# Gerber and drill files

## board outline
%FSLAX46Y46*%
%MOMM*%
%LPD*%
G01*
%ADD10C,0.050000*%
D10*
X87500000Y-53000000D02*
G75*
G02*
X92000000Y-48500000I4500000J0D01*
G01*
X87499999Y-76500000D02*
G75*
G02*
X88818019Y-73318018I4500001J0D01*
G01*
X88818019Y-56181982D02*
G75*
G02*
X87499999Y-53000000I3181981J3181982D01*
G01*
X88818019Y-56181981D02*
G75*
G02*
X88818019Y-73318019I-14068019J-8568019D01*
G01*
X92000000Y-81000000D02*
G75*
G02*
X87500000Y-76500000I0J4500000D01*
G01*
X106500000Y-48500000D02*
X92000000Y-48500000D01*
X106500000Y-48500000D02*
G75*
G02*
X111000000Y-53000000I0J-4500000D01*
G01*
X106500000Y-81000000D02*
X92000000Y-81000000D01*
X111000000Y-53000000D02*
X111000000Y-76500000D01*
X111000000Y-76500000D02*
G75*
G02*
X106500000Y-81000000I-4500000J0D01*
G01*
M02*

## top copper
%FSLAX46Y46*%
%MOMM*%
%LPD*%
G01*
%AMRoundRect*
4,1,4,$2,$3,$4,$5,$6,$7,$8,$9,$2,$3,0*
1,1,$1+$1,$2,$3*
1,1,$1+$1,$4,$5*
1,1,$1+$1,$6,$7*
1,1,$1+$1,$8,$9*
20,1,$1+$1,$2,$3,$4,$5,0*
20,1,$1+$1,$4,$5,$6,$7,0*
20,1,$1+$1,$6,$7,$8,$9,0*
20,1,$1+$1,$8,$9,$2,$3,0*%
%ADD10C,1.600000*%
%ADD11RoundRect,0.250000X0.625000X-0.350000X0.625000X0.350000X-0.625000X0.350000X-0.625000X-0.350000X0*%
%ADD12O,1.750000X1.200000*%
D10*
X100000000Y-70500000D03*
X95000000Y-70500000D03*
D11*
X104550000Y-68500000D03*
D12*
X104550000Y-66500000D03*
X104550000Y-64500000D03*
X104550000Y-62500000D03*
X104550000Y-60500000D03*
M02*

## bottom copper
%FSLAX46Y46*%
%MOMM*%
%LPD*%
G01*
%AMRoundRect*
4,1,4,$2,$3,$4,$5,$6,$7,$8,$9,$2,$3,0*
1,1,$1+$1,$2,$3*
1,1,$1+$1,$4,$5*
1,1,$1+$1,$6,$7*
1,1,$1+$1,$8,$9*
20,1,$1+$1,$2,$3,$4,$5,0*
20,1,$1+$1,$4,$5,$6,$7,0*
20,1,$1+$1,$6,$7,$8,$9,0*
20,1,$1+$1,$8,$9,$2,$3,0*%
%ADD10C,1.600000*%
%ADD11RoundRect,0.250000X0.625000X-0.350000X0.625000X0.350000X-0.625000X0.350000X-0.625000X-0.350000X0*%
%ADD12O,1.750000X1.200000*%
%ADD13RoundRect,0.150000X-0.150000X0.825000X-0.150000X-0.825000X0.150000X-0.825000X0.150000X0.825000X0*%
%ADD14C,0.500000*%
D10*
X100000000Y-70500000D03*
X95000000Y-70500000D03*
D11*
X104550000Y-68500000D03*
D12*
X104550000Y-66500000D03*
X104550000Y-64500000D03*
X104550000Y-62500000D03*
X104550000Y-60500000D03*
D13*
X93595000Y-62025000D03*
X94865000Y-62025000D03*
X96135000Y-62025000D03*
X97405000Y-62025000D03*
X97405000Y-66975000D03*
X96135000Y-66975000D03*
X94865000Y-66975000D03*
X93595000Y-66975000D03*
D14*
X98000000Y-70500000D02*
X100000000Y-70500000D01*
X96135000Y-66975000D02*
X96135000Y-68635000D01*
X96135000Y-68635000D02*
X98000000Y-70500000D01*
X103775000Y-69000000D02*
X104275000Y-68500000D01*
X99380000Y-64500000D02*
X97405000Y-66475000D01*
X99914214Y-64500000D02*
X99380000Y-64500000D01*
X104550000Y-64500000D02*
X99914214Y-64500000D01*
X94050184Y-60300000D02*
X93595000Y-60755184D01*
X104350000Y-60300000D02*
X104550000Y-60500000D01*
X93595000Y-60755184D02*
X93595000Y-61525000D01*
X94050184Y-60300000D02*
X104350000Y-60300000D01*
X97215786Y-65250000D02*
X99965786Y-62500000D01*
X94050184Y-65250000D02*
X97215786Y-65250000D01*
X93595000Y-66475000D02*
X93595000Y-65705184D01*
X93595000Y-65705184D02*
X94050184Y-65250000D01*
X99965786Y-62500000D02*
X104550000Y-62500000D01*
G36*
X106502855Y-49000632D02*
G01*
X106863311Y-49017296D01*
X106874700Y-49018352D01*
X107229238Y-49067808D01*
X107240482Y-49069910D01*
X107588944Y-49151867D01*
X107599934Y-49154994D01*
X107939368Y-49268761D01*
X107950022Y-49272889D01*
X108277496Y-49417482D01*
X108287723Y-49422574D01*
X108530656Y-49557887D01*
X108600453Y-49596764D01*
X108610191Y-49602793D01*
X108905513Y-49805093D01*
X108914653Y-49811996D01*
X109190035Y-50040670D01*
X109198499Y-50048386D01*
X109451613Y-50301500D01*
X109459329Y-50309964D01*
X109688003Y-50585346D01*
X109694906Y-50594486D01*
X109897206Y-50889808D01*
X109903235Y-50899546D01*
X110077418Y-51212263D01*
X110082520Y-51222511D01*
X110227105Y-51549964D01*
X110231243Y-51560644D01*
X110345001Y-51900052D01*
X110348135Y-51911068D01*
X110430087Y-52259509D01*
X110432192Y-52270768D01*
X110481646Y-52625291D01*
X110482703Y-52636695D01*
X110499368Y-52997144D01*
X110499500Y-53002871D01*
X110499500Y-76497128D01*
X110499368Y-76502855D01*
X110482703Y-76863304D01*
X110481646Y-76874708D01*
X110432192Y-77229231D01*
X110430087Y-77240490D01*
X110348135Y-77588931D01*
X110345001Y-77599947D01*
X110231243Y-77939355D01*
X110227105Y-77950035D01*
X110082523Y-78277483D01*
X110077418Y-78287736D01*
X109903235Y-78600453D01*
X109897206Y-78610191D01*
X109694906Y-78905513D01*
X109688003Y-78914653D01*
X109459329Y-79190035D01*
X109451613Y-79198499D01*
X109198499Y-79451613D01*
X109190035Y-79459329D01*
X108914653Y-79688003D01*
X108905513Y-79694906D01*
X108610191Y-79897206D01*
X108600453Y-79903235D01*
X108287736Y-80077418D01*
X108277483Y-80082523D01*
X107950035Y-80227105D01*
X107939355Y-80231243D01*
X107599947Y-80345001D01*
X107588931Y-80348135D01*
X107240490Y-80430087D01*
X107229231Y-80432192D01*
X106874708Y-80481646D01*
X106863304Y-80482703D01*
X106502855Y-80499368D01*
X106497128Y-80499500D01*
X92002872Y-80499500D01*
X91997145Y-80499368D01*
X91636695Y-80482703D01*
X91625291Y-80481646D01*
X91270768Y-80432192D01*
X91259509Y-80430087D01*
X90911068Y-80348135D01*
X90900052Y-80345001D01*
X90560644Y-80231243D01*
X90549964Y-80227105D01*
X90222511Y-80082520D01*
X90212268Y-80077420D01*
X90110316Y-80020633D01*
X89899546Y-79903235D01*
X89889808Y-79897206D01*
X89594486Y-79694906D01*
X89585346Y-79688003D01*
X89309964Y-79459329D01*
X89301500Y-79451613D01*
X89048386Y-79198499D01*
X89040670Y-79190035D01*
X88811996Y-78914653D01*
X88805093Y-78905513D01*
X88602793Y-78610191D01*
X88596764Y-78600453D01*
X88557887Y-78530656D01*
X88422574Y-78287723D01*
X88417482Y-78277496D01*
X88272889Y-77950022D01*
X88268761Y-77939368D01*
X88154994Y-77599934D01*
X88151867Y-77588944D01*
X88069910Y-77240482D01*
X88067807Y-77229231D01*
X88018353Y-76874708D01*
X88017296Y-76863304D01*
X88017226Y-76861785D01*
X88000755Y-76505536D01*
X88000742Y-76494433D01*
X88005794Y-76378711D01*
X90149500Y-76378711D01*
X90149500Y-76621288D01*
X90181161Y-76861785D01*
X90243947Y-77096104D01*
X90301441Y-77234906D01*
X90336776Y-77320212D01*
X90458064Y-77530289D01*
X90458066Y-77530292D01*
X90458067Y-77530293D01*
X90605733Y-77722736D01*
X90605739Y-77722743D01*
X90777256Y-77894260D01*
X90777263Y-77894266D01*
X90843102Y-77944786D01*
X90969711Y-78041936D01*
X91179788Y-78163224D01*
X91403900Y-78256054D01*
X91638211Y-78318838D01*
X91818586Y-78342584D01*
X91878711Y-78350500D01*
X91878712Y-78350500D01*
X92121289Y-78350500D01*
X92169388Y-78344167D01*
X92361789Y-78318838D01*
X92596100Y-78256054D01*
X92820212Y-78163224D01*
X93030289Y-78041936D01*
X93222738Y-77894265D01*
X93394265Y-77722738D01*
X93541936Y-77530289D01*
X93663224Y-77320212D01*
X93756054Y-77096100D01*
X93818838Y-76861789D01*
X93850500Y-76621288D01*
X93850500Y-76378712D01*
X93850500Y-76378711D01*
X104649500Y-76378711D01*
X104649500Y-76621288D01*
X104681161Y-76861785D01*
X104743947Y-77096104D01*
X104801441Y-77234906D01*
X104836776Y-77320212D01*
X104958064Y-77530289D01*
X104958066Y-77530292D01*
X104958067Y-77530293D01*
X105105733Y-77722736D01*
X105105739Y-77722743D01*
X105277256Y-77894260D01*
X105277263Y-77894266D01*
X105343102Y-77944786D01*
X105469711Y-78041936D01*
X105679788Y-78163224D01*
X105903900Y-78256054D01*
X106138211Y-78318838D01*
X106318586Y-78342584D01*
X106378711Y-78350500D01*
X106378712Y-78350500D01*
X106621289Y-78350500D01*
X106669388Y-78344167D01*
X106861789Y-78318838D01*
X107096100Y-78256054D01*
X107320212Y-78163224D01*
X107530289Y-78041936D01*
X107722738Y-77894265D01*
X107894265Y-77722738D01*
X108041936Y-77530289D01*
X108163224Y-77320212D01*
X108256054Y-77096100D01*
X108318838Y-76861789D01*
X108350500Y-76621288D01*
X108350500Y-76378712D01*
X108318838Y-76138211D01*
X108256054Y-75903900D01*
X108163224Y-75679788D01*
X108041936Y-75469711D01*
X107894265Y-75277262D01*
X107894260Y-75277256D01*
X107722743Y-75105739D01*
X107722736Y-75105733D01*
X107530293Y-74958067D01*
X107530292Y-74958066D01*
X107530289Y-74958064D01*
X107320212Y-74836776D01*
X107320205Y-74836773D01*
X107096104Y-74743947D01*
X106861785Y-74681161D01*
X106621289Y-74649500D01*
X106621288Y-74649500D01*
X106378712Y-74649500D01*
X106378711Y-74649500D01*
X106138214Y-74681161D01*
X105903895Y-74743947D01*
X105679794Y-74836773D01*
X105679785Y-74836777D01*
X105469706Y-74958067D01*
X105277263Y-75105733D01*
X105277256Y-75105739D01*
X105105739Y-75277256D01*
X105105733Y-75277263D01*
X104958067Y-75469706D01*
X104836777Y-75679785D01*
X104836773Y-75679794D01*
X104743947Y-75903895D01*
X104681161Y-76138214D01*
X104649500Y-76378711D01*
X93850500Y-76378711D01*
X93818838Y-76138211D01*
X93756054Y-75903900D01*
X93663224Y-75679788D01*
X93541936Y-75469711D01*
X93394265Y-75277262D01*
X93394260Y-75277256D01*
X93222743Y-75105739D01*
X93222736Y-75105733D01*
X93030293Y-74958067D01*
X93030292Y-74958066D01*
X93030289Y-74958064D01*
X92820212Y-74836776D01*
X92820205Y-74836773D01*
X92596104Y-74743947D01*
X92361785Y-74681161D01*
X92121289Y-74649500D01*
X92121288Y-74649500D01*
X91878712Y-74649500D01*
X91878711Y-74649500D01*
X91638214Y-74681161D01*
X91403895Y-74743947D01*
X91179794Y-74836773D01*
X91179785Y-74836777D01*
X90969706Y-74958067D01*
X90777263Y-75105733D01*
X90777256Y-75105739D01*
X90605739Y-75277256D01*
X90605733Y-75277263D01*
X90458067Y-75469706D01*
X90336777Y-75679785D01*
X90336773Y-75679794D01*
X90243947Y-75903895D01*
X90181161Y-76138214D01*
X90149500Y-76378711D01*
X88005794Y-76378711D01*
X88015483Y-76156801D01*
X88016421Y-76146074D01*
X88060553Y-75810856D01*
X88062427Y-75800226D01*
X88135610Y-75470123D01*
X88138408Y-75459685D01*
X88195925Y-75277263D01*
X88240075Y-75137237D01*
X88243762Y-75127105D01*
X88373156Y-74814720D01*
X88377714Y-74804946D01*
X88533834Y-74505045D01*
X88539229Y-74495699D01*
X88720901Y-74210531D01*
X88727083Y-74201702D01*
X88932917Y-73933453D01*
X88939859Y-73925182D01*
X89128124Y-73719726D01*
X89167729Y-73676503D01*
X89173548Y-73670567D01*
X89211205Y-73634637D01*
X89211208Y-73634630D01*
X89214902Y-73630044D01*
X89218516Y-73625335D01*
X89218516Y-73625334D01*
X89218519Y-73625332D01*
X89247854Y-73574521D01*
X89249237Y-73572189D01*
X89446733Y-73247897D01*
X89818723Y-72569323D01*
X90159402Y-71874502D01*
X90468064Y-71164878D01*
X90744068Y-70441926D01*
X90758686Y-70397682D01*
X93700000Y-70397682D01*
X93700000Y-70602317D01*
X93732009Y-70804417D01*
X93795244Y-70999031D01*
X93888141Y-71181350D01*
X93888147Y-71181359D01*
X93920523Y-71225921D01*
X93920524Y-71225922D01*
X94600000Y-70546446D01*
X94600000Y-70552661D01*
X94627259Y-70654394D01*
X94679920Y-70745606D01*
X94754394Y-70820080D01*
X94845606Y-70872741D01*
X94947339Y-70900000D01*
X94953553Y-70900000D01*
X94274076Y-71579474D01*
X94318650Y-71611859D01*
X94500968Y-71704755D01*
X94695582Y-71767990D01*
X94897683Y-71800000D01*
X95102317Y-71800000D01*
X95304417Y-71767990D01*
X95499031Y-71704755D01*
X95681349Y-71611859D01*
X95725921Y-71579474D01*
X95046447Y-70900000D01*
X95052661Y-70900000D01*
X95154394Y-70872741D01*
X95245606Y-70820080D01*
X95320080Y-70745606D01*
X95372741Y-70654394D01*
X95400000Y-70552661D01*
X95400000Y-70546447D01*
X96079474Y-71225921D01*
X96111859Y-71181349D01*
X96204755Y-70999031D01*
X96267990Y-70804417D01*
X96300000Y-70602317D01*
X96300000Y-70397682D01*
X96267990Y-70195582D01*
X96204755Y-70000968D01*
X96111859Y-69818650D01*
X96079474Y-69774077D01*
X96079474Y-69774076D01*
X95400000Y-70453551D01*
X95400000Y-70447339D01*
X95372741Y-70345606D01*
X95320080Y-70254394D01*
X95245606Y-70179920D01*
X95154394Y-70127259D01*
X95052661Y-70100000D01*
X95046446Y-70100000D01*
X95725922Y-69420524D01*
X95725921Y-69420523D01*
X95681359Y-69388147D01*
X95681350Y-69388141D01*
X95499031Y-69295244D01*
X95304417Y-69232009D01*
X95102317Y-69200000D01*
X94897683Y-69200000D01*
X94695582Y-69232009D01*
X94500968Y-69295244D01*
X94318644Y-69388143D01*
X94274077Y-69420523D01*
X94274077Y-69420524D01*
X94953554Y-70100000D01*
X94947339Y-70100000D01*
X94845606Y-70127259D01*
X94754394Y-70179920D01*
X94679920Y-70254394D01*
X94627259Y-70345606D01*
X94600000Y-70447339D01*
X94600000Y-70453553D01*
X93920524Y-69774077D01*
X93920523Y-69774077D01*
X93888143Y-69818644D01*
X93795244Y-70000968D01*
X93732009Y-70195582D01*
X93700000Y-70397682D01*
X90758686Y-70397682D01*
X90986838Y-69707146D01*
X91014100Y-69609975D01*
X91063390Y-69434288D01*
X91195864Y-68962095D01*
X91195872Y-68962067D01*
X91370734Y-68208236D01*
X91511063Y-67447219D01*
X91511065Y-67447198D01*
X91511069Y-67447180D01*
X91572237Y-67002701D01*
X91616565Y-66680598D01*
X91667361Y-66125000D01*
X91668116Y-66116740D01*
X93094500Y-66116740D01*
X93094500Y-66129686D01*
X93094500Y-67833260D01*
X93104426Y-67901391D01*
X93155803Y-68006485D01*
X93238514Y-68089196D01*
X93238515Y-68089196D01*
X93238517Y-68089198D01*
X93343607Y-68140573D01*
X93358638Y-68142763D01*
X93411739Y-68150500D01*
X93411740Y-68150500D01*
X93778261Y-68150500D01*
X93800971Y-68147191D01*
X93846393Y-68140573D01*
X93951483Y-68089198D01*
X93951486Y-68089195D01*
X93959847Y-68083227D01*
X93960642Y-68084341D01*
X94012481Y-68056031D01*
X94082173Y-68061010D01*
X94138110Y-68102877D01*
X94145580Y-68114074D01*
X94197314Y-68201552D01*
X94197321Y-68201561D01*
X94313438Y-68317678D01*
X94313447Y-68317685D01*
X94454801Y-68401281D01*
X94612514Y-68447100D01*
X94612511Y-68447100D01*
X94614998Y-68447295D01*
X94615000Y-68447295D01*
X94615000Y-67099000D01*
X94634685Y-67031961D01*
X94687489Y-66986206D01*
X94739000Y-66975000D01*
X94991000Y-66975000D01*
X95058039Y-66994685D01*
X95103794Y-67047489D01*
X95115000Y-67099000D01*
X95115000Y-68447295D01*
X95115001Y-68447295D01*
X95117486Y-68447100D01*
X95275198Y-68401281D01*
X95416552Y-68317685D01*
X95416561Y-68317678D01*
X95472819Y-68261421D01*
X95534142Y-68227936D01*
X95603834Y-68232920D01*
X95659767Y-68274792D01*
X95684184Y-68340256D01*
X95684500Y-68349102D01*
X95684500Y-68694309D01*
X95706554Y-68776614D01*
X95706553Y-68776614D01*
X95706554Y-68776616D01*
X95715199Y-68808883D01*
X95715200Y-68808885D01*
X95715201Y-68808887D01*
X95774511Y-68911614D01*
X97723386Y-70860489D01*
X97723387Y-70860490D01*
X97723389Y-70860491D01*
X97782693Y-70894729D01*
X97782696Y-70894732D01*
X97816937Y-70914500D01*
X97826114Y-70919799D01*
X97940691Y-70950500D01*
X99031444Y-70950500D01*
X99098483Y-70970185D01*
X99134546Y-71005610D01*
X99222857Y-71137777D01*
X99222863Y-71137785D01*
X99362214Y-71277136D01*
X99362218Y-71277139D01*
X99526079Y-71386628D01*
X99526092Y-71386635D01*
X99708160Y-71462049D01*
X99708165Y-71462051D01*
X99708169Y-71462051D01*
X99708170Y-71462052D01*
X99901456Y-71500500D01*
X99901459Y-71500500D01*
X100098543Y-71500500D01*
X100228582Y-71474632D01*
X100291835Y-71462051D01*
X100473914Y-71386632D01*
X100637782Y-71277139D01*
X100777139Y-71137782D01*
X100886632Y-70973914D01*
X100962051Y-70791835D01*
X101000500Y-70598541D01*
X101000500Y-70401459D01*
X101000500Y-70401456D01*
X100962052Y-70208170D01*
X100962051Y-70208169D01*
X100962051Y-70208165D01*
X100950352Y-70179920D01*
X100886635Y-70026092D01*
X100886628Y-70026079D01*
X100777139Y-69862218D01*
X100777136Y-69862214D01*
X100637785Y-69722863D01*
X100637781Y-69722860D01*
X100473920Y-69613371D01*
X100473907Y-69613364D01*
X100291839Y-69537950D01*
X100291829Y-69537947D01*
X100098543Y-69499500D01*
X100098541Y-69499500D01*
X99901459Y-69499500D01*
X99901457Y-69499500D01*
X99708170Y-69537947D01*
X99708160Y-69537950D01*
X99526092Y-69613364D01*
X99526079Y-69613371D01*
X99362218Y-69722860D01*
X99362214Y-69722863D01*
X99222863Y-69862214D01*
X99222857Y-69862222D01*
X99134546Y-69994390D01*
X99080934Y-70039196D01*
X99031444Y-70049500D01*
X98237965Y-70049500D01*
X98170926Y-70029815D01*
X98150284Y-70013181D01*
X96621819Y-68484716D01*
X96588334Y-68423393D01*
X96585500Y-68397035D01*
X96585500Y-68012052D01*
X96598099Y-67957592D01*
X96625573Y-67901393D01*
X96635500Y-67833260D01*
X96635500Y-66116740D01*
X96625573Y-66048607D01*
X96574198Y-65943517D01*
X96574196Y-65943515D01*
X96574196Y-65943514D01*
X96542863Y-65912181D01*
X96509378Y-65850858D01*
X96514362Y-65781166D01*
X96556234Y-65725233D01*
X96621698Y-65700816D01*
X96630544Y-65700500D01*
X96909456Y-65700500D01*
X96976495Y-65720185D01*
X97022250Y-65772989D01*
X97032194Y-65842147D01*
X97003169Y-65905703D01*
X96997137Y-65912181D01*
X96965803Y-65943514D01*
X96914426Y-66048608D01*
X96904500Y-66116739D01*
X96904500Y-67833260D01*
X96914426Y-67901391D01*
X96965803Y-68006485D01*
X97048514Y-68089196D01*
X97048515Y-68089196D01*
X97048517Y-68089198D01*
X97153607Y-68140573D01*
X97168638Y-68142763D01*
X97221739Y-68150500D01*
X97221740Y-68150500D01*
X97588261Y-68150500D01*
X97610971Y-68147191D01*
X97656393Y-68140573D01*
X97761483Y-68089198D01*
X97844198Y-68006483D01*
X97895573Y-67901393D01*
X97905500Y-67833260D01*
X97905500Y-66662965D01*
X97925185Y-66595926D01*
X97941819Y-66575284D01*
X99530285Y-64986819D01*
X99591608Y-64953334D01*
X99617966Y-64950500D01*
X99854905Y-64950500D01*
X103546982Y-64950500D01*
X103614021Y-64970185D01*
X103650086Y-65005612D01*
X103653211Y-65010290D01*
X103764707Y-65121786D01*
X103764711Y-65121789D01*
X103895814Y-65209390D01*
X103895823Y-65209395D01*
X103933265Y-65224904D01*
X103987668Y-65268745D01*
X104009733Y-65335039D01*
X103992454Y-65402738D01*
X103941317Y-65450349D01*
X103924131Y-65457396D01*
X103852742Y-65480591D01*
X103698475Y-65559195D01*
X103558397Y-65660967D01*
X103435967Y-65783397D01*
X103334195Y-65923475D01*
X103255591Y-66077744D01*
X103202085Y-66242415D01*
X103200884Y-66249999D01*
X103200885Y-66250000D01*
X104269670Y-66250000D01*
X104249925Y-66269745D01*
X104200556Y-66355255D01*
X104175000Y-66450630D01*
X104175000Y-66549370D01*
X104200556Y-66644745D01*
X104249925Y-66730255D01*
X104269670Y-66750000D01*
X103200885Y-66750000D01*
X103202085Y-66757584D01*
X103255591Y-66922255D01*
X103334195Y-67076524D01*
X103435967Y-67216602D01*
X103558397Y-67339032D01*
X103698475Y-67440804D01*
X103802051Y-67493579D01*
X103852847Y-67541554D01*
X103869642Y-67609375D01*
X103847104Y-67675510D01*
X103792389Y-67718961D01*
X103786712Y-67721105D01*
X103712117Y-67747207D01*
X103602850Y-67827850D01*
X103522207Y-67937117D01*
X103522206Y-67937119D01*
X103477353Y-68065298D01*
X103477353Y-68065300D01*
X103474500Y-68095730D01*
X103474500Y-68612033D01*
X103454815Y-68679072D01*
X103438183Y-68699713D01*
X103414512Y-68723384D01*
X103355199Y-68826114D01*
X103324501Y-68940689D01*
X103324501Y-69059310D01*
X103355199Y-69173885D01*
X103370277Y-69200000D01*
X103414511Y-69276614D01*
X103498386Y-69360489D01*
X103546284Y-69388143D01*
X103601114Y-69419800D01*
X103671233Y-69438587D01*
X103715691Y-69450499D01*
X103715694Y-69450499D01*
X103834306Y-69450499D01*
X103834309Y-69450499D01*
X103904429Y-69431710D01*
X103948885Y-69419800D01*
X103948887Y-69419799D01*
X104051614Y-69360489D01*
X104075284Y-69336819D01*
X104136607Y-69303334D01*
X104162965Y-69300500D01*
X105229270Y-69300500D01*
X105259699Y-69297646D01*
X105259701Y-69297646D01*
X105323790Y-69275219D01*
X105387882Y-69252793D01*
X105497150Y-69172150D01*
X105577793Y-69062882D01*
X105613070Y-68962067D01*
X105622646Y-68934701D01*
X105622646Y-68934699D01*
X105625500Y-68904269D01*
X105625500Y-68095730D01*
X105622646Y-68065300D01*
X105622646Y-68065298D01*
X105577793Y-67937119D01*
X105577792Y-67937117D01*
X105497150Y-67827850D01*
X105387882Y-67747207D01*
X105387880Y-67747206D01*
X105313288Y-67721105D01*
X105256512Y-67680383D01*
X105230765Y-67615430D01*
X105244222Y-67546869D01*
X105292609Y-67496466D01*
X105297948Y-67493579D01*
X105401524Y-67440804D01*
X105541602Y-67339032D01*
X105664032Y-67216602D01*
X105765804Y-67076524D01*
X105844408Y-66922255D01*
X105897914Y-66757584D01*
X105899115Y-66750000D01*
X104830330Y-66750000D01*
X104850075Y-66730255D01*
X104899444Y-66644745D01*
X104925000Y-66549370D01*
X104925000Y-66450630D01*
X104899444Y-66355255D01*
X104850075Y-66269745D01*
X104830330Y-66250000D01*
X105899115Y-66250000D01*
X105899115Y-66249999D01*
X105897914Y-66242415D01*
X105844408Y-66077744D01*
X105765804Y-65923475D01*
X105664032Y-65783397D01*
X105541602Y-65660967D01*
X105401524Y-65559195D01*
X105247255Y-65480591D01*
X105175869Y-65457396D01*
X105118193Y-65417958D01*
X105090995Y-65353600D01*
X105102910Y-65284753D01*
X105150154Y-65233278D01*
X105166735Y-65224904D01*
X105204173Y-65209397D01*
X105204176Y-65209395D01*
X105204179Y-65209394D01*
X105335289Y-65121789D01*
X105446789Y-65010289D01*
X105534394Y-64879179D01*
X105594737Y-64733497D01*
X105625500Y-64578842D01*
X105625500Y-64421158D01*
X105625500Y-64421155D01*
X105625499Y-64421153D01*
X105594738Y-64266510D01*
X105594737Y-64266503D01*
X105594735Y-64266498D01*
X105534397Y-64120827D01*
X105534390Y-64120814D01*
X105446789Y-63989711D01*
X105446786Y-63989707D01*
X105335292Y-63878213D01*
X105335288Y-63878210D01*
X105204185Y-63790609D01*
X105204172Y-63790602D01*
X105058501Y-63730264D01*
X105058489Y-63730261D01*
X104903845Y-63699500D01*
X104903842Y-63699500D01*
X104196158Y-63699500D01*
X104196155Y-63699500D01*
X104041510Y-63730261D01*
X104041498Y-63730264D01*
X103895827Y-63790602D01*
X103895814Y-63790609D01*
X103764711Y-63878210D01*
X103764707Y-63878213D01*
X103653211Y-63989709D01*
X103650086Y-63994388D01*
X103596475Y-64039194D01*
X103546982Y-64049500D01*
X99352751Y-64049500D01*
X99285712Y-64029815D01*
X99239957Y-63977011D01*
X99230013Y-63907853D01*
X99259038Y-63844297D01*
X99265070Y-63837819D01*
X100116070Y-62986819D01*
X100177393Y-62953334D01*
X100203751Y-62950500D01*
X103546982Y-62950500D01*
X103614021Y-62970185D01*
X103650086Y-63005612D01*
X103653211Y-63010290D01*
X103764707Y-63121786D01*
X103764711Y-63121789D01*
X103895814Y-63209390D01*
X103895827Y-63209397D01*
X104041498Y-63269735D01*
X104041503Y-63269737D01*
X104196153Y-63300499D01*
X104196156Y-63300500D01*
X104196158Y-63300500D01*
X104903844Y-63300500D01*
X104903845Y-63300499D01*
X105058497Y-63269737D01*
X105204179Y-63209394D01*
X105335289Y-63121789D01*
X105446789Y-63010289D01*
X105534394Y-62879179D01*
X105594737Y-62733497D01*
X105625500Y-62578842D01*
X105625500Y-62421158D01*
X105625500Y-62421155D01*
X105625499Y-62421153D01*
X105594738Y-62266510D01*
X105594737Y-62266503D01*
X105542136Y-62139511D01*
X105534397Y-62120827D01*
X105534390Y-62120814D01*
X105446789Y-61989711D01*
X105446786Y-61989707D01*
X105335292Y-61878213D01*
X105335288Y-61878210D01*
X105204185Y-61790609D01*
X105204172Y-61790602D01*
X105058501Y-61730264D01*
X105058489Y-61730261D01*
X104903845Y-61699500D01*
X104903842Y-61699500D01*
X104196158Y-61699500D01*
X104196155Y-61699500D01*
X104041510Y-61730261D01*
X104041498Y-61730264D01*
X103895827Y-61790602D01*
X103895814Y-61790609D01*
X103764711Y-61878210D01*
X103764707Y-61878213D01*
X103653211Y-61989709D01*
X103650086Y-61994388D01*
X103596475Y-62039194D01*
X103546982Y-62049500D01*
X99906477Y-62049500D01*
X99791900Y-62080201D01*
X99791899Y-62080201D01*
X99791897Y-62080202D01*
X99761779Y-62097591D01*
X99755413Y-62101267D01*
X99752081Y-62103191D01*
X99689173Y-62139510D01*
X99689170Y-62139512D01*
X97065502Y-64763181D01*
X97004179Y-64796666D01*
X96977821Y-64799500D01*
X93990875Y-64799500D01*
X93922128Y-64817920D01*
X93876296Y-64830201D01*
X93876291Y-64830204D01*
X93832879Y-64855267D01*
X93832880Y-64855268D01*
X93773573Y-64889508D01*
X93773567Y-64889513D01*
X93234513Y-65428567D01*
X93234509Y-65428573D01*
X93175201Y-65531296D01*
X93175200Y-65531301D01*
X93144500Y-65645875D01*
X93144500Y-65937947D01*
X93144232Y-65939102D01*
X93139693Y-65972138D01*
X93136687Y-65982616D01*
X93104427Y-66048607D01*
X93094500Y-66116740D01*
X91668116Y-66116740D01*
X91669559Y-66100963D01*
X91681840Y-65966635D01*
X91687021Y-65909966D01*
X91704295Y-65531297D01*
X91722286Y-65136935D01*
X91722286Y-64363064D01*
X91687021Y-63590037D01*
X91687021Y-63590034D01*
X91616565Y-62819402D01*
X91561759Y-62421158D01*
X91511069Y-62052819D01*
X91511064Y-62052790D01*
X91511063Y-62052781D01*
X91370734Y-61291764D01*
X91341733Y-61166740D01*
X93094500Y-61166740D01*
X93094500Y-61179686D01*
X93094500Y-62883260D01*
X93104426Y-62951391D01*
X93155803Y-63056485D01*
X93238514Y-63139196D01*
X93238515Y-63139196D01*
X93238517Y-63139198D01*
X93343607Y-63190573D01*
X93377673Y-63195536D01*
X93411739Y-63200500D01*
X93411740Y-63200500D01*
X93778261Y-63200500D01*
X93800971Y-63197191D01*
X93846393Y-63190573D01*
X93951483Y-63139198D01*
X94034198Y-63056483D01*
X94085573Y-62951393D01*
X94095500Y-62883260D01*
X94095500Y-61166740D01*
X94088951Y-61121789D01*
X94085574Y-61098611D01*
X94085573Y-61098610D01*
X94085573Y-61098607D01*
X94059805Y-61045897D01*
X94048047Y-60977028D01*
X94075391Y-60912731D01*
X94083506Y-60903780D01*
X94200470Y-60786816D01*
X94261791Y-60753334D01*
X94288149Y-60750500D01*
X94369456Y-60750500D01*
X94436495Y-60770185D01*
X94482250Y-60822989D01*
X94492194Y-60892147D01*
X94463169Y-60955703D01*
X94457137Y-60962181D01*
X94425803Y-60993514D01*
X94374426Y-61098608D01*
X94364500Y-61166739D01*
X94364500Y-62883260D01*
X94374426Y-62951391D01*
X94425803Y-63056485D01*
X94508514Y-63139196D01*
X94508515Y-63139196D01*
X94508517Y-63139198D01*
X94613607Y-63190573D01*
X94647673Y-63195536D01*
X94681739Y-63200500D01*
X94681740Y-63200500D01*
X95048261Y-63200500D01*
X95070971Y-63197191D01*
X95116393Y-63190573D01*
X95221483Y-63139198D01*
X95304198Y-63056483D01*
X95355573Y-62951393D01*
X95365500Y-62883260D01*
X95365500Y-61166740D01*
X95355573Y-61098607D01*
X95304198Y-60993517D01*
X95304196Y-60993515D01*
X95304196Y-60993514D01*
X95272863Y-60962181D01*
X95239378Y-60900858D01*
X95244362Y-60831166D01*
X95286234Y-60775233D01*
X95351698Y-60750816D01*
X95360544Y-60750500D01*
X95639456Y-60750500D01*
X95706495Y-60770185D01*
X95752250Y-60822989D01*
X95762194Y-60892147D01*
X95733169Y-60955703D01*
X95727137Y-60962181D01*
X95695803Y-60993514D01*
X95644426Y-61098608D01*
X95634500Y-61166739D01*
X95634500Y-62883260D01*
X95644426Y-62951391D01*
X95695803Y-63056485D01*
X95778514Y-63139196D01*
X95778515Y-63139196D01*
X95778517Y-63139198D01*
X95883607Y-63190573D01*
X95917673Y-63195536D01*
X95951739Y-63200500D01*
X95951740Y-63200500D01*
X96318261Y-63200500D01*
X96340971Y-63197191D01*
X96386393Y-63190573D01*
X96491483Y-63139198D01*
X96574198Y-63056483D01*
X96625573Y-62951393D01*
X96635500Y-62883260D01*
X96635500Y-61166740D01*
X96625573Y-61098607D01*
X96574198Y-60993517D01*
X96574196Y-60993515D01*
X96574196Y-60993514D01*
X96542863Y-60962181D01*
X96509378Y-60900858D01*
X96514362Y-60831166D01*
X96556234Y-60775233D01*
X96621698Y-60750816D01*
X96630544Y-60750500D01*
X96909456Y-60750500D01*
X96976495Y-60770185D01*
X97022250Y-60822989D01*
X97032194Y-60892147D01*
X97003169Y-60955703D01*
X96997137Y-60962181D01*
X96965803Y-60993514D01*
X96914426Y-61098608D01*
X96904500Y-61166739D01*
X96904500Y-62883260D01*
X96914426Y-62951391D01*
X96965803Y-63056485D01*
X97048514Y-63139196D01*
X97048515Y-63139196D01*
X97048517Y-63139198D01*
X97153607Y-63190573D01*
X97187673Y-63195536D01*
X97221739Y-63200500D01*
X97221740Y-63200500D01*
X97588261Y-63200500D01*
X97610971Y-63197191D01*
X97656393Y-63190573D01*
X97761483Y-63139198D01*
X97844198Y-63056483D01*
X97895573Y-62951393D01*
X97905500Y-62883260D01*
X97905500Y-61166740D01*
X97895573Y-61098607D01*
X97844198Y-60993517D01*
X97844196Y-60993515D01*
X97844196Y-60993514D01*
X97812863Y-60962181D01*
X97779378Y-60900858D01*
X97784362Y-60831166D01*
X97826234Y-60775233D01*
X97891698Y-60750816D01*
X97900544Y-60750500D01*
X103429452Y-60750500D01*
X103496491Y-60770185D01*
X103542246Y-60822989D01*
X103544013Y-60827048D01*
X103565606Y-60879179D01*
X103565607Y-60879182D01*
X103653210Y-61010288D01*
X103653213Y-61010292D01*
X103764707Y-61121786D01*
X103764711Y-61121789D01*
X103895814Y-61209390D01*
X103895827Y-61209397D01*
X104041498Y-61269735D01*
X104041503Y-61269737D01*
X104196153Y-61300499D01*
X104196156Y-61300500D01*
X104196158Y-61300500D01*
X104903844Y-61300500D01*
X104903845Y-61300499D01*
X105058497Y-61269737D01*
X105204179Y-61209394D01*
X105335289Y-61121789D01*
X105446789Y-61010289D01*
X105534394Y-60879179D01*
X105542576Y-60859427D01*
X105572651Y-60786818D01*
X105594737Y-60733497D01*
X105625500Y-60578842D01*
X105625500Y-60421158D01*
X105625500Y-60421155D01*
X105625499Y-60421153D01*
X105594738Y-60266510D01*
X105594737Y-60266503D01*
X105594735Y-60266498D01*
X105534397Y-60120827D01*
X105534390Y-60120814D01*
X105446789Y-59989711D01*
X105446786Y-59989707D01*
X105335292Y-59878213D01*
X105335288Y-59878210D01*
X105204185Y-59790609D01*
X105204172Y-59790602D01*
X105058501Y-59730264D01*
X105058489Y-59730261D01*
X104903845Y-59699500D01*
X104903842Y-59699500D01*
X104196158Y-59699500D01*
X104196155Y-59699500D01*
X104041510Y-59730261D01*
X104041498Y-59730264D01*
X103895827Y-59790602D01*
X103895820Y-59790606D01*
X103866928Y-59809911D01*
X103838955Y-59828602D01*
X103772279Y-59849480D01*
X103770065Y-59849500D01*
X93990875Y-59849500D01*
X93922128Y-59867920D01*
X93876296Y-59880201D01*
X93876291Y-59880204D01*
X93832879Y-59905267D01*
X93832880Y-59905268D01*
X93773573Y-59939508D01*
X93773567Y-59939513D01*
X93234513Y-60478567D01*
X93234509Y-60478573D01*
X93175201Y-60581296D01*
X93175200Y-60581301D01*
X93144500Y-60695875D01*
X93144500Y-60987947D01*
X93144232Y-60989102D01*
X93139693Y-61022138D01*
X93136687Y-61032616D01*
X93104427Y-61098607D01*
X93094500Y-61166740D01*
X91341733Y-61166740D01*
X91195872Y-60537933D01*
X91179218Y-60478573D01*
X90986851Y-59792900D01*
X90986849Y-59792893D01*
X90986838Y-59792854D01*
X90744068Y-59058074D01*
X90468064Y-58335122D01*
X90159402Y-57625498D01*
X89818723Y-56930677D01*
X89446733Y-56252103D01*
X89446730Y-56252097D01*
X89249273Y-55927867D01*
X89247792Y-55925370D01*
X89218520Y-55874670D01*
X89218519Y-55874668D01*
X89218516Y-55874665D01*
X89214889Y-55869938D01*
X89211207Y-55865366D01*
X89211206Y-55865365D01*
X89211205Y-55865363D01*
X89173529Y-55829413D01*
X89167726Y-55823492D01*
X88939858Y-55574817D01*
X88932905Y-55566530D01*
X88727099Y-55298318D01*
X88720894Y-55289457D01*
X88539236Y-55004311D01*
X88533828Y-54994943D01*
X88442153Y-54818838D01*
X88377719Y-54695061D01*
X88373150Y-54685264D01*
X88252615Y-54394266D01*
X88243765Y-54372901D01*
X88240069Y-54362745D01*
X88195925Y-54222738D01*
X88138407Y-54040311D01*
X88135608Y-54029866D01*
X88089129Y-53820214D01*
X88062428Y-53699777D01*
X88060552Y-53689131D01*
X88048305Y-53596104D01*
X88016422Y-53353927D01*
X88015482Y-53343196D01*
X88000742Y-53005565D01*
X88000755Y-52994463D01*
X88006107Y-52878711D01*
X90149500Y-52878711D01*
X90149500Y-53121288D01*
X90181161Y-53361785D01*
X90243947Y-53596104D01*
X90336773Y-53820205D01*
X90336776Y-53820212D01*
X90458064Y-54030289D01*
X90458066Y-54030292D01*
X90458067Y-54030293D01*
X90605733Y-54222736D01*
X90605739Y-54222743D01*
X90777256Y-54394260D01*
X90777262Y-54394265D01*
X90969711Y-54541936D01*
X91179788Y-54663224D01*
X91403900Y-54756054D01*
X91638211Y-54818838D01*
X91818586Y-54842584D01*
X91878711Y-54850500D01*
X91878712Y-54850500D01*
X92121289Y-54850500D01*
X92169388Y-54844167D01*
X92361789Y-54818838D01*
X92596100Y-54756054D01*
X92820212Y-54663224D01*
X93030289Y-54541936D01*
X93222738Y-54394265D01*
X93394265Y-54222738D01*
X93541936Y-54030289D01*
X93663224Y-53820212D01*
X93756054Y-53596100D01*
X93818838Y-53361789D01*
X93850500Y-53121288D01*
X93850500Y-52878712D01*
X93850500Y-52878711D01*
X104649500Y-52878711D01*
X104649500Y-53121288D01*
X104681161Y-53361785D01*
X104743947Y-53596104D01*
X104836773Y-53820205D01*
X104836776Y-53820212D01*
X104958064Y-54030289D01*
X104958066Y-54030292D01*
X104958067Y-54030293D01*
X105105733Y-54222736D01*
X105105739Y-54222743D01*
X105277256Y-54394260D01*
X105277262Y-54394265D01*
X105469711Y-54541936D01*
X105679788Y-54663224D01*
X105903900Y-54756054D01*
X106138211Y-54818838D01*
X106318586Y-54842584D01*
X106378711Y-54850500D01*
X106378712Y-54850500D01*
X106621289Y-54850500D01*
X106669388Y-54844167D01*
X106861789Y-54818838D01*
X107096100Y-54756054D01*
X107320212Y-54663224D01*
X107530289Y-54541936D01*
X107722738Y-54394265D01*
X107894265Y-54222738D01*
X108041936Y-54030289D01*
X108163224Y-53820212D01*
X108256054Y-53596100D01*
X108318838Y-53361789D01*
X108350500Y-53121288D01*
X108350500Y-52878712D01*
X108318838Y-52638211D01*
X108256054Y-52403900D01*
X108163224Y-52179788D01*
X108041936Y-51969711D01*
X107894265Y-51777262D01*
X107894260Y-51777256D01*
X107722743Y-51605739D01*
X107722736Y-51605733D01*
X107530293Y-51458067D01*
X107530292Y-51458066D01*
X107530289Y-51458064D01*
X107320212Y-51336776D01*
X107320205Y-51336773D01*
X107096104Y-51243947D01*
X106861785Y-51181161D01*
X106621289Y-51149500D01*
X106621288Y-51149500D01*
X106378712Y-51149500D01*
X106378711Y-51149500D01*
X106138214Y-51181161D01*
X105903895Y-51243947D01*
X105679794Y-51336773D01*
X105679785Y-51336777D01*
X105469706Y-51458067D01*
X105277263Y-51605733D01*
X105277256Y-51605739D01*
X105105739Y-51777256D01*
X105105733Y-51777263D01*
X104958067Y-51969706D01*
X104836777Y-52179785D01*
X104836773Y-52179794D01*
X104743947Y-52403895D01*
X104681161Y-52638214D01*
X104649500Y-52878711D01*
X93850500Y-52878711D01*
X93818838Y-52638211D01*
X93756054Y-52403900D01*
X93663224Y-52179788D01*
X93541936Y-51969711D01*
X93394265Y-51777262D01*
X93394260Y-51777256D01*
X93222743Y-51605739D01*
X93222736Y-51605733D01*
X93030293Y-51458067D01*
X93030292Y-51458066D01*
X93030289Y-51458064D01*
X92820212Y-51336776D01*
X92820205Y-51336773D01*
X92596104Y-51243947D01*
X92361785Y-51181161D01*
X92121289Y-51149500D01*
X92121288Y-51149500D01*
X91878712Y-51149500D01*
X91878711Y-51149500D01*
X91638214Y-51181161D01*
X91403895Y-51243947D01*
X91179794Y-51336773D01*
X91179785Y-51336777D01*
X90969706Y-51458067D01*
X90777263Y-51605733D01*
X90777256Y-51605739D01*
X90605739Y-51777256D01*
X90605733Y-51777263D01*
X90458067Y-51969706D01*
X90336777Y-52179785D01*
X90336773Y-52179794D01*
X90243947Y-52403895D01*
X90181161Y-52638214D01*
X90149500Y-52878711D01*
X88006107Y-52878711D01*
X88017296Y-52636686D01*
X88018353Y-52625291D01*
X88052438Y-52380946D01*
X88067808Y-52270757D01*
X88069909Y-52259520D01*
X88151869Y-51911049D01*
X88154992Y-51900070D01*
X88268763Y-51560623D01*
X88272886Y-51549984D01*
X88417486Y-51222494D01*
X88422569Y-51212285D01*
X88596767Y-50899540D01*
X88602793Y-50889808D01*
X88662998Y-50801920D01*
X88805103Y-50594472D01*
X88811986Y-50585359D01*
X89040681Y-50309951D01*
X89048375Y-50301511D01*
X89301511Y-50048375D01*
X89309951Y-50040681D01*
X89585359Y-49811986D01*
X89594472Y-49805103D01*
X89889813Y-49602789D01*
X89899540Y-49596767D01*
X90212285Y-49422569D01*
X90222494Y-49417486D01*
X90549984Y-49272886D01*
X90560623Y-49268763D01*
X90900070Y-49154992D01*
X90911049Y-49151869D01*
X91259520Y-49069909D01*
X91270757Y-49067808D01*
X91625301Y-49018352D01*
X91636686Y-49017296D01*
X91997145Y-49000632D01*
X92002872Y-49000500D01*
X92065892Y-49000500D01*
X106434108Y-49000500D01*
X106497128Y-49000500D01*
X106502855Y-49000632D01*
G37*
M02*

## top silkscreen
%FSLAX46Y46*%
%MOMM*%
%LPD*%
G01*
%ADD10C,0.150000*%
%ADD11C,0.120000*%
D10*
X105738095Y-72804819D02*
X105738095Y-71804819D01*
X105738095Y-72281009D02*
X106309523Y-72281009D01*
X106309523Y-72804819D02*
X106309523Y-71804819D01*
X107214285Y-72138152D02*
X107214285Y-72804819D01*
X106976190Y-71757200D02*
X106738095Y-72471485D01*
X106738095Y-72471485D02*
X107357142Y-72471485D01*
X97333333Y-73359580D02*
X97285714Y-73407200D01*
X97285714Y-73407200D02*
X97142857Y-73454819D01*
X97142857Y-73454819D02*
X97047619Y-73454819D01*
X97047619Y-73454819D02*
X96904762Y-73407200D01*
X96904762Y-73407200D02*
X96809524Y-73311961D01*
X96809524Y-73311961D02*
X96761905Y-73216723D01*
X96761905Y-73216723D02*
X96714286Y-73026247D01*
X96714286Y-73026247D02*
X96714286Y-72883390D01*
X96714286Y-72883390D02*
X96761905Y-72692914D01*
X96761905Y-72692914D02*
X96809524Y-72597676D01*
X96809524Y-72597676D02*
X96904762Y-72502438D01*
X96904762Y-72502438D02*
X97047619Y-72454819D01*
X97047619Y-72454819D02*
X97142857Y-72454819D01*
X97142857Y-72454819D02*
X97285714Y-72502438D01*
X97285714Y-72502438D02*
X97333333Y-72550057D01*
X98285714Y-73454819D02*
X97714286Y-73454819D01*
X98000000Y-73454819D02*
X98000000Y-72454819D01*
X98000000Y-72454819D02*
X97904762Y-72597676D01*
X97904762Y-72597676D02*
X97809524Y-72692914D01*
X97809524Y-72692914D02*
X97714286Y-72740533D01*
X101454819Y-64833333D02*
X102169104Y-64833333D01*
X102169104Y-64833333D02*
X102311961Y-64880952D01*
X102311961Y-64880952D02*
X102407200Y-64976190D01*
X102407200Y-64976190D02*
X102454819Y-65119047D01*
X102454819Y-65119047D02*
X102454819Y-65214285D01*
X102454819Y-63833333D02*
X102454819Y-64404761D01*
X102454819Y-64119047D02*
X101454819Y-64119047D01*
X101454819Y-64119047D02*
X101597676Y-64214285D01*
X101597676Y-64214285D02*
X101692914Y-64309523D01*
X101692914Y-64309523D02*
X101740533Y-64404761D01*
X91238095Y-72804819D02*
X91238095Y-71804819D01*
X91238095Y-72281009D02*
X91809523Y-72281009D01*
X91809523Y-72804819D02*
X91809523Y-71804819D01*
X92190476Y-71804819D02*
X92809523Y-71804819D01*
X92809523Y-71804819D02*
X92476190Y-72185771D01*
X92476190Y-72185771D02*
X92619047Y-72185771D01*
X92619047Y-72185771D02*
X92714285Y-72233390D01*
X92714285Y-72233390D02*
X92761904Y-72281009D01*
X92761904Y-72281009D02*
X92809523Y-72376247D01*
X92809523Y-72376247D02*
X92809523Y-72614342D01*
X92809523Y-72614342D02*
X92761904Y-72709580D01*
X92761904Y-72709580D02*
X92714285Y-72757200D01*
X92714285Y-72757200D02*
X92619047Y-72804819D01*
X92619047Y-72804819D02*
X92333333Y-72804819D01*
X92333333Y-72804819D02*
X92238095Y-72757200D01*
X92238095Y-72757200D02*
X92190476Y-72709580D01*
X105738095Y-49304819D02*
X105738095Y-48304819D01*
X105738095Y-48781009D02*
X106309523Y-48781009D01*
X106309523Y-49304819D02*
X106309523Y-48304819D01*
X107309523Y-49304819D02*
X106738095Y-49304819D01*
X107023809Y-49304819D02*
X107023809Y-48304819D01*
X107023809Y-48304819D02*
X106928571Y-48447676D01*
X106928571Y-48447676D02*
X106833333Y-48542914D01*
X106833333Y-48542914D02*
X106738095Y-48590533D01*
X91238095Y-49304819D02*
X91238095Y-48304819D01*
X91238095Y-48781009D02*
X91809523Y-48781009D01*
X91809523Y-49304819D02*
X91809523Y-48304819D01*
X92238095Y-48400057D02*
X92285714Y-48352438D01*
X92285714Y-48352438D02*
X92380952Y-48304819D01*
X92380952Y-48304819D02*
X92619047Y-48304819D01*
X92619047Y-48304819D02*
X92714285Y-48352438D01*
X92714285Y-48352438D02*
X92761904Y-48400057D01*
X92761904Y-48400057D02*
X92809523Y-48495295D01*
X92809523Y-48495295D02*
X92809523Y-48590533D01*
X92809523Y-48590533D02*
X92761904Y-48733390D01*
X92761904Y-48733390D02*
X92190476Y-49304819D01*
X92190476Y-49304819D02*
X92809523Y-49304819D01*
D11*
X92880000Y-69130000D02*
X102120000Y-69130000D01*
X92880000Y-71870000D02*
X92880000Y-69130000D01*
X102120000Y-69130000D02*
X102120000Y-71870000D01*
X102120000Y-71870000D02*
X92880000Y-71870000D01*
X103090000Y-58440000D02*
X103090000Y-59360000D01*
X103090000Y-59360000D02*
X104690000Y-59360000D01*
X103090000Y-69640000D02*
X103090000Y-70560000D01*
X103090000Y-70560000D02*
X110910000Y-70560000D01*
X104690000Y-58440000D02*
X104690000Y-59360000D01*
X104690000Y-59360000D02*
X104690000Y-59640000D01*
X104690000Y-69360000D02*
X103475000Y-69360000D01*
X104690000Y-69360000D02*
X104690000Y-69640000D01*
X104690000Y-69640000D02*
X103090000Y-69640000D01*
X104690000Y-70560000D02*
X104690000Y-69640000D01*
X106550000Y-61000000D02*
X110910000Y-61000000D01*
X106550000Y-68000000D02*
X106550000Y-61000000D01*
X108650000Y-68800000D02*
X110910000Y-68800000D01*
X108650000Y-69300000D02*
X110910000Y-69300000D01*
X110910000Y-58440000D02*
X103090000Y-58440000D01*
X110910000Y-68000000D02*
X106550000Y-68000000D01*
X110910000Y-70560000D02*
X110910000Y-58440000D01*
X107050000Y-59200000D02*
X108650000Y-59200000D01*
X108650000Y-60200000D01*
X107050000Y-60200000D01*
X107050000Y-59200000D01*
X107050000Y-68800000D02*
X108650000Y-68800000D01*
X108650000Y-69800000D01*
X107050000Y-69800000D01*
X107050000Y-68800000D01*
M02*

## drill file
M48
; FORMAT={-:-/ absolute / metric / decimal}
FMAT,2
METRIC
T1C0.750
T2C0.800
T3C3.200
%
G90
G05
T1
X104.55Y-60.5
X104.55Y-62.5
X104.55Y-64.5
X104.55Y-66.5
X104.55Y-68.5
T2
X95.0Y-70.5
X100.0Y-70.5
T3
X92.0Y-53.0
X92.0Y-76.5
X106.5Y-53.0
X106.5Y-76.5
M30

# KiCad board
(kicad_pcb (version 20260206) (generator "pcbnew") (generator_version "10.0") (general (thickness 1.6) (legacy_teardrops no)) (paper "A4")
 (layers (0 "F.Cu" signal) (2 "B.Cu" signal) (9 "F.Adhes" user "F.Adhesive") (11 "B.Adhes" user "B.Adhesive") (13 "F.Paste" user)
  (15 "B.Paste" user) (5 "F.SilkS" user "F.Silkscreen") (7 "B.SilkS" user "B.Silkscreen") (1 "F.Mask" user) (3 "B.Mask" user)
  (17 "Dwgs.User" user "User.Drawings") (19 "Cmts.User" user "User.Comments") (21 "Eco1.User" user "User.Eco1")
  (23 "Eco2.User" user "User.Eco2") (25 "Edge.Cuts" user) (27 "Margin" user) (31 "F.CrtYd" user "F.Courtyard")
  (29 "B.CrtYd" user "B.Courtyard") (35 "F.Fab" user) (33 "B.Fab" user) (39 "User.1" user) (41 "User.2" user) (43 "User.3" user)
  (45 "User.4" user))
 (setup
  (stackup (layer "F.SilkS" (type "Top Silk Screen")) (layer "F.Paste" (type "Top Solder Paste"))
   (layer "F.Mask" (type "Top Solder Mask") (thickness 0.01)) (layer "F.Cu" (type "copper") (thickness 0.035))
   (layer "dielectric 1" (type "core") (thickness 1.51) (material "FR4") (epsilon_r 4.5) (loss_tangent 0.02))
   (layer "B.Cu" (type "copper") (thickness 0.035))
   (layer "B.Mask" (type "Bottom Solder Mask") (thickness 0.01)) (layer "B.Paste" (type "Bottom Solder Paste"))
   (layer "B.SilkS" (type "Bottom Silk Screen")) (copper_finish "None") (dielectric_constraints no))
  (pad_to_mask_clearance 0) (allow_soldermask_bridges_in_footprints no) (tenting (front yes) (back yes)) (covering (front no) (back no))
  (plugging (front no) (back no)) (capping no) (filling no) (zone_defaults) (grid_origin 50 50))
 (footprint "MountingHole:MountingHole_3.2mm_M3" (layer "F.Cu") (at 106.5 76.5)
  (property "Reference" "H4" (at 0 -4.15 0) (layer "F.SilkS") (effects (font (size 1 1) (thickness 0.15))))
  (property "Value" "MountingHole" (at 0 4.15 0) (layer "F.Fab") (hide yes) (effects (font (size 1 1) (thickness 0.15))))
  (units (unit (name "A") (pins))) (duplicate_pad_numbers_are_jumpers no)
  (pad "" np_thru_hole circle (at 0 0) (size 3.2 3.2) (drill 3.2) (layers "*.Cu" "*.Mask")))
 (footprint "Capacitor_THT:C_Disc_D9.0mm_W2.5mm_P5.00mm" (layer "F.Cu") (at 100 70.5 180)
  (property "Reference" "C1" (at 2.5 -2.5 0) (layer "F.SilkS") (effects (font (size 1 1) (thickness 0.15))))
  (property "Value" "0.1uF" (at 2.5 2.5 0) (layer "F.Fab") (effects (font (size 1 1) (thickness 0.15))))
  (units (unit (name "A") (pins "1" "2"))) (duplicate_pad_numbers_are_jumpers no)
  (fp_line (start 7.12 1.37) (end -2.12 1.37) (stroke (width 0.12) (type solid)) (layer "F.SilkS"))
  (fp_line (start 7.12 -1.37) (end 7.12 1.37) (stroke (width 0.12) (type solid)) (layer "F.SilkS"))
  (fp_line (start -2.12 1.37) (end -2.12 -1.37) (stroke (width 0.12) (type solid)) (layer "F.SilkS"))
  (fp_line (start -2.12 -1.37) (end 7.12 -1.37) (stroke (width 0.12) (type solid)) (layer "F.SilkS"))
  (pad "1" thru_hole circle (at 0 0 180) (size 1.6 1.6) (drill 0.8) (layers "*.Cu" "*.Mask") (remove_unused_layers no) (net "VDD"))
  (pad "2" thru_hole circle (at 5 0 180) (size 1.6 1.6) (drill 0.8) (layers "*.Cu" "*.Mask") (remove_unused_layers no) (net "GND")))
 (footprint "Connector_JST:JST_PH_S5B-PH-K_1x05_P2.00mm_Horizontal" (layer "F.Cu") (at 104.55 68.5 90)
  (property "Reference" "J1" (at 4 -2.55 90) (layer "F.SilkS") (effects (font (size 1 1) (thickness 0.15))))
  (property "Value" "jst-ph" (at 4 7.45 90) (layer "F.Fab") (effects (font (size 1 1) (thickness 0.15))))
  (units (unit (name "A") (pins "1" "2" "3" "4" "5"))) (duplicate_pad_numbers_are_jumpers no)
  (fp_line (start 10.06 -1.46) (end 9.14 -1.46) (stroke (width 0.12) (type solid)) (layer "F.SilkS"))
  (fp_line (start 9.14 -1.46) (end 9.14 0.14) (stroke (width 0.12) (type solid)) (layer "F.SilkS"))
  (fp_line (start -1.14 -1.46) (end -2.06 -1.46) (stroke (width 0.12) (type solid)) (layer "F.SilkS"))
  (fp_line (start -2.06 -1.46) (end -2.06 6.36) (stroke (width 0.12) (type solid)) (layer "F.SilkS"))
  (fp_line (start 10.06 0.14) (end 9.14 0.14) (stroke (width 0.12) (type solid)) (layer "F.SilkS"))
  (fp_line (start 9.14 0.14) (end 8.86 0.14) (stroke (width 0.12) (type solid)) (layer "F.SilkS"))
  (fp_line (start -0.86 0.14) (end -0.86 -1.075) (stroke (width 0.12) (type solid)) (layer "F.SilkS"))
  (fp_line (start -0.86 0.14) (end -1.14 0.14) (stroke (width 0.12) (type solid)) (layer "F.SilkS"))
  (fp_line (start -1.14 0.14) (end -1.14 -1.46) (stroke (width 0.12) (type solid)) (layer "F.SilkS"))
  (fp_line (start -2.06 0.14) (end -1.14 0.14) (stroke (width 0.12) (type solid)) (layer "F.SilkS"))
  (fp_line (start 7.5 2) (end 7.5 6.36) (stroke (width 0.12) (type solid)) (layer "F.SilkS"))
  (fp_line (start 0.5 2) (end 7.5 2) (stroke (width 0.12) (type solid)) (layer "F.SilkS"))
  (fp_line (start -0.3 4.1) (end -0.3 6.36) (stroke (width 0.12) (type solid)) (layer "F.SilkS"))
  (fp_line (start -0.8 4.1) (end -0.8 6.36) (stroke (width 0.12) (type solid)) (layer "F.SilkS"))
  (fp_line (start 10.06 6.36) (end 10.06 -1.46) (stroke (width 0.12) (type solid)) (layer "F.SilkS"))
  (fp_line (start 0.5 6.36) (end 0.5 2) (stroke (width 0.12) (type solid)) (layer "F.SilkS"))
  (fp_line (start -2.06 6.36) (end 10.06 6.36) (stroke (width 0.12) (type solid)) (layer "F.SilkS"))
  (fp_rect (start 8.3 2.5) (end 9.3 4.1) (stroke (width 0.12) (type solid)) (fill no) (layer "F.SilkS"))
  (fp_rect (start -1.3 2.5) (end -0.3 4.1) (stroke (width 0.12) (type solid)) (fill no) (layer "F.SilkS"))
  (pad "1" thru_hole roundrect (at 0 0 90) (size 1.2 1.75) (drill 0.75) (layers "*.Cu" "*.Mask") (remove_unused_layers no)
   (roundrect_rratio 0.208333) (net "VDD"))
  (pad "2" thru_hole oval (at 2 0 90) (size 1.2 1.75) (drill 0.75) (layers "*.Cu" "*.Mask") (remove_unused_layers no) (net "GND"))
  (pad "3" thru_hole oval (at 4 0 90) (size 1.2 1.75) (drill 0.75) (layers "*.Cu" "*.Mask") (remove_unused_layers no) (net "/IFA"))
  (pad "4" thru_hole oval (at 6 0 90) (size 1.2 1.75) (drill 0.75) (layers "*.Cu" "*.Mask") (remove_unused_layers no) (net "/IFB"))
  (pad "5" thru_hole oval (at 8 0 90) (size 1.2 1.75) (drill 0.75) (layers "*.Cu" "*.Mask") (remove_unused_layers no) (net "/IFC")))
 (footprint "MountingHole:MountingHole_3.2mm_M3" (layer "F.Cu") (at 92 76.5)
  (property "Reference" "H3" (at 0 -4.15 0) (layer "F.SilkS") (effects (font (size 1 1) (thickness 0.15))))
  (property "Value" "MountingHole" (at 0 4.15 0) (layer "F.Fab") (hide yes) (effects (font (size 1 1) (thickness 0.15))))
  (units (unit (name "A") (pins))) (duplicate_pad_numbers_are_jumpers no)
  (pad "" np_thru_hole circle (at 0 0) (size 3.2 3.2) (drill 3.2) (layers "*.Cu" "*.Mask")))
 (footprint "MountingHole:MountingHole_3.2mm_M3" (layer "F.Cu") (at 106.5 53)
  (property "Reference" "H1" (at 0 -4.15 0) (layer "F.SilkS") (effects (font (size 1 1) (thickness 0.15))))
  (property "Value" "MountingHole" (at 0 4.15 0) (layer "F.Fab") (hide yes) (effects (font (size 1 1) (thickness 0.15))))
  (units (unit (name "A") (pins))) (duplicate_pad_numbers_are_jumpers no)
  (pad "" np_thru_hole circle (at 0 0) (size 3.2 3.2) (drill 3.2) (layers "*.Cu" "*.Mask")))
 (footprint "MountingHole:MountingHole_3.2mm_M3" (layer "F.Cu") (at 92 53)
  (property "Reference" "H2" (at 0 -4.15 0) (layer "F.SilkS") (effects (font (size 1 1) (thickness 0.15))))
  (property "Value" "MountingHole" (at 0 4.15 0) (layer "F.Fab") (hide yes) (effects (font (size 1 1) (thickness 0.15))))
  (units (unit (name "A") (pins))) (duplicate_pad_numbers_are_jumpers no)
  (pad "" np_thru_hole circle (at 0 0) (size 3.2 3.2) (drill 3.2) (layers "*.Cu" "*.Mask")))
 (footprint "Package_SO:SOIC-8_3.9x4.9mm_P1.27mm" (layer "B.Cu") (at 95.5 64.5 -90)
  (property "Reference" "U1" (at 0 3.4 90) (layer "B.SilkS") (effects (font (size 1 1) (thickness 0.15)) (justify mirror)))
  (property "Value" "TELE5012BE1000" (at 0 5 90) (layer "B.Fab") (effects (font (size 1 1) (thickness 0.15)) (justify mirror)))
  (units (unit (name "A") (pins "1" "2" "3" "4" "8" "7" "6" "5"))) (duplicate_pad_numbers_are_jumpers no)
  (pad "1" smd roundrect (at -2.475 1.905 270) (size 1.95 0.6) (layers "B.Cu" "B.Mask" "B.Paste") (roundrect_rratio 0.25) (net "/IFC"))
  (pad "2" smd roundrect (at -2.475 0.635 270) (size 1.95 0.6) (layers "B.Cu" "B.Mask" "B.Paste") (roundrect_rratio 0.25)
   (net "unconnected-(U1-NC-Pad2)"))
  (pad "3" smd roundrect (at -2.475 -0.635 270) (size 1.95 0.6) (layers "B.Cu" "B.Mask" "B.Paste") (roundrect_rratio 0.25)
   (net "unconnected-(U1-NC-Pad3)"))
  (pad "4" smd roundrect (at -2.475 -1.905 270) (size 1.95 0.6) (layers "B.Cu" "B.Mask" "B.Paste") (roundrect_rratio 0.25)
   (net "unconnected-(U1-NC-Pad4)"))
  (pad "5" smd roundrect (at 2.475 -1.905 270) (size 1.95 0.6) (layers "B.Cu" "B.Mask" "B.Paste") (roundrect_rratio 0.25) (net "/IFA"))
  (pad "6" smd roundrect (at 2.475 -0.635 270) (size 1.95 0.6) (layers "B.Cu" "B.Mask" "B.Paste") (roundrect_rratio 0.25) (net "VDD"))
  (pad "7" smd roundrect (at 2.475 0.635 270) (size 1.95 0.6) (layers "B.Cu" "B.Mask" "B.Paste") (roundrect_rratio 0.25) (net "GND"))
  (pad "8" smd roundrect (at 2.475 1.905 270) (size 1.95 0.6) (layers "B.Cu" "B.Mask" "B.Paste") (roundrect_rratio 0.25) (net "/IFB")))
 (gr_arc (start 87.5 53) (mid 88.818019 49.818019) (end 92 48.5) (stroke (width 0.05) (type default)) (layer "Edge.Cuts"))
 (gr_arc (start 87.499999 76.5) (mid 87.842541 74.777924) (end 88.818019 73.318018) (stroke (width 0.05) (type default)) (layer "Edge.Cuts"))
 (gr_arc (start 88.818019 56.181982) (mid 87.842541 54.722076) (end 87.499999 53) (stroke (width 0.05) (type default)) (layer "Edge.Cuts"))
 (gr_arc (start 88.818019 56.181981) (mid 91.221797 64.75) (end 88.818019 73.318019) (stroke (width 0.05) (type default))
  (layer "Edge.Cuts"))
 (gr_arc (start 92 81) (mid 88.818019 79.681981) (end 87.5 76.5) (stroke (width 0.05) (type default)) (layer "Edge.Cuts"))
 (gr_line (start 106.5 48.5) (end 92 48.5) (stroke (width 0.05) (type default)) (layer "Edge.Cuts"))
 (gr_arc (start 106.5 48.5) (mid 109.681981 49.818019) (end 111 53) (stroke (width 0.05) (type default)) (layer "Edge.Cuts"))
 (gr_line (start 106.5 81) (end 92 81) (stroke (width 0.05) (type default)) (layer "Edge.Cuts"))
 (gr_line (start 111 53) (end 111 76.5) (stroke (width 0.05) (type default)) (layer "Edge.Cuts"))
 (gr_arc (start 111 76.5) (mid 109.681981 79.681981) (end 106.5 81) (stroke (width 0.05) (type default)) (layer "Edge.Cuts"))
 (segment (start 98 70.5) (end 100 70.5) (width 0.5) (layer "B.Cu") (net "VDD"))
 (segment (start 96.135 66.975) (end 96.135 68.635) (width 0.5) (layer "B.Cu") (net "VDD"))
 (segment (start 96.135 68.635) (end 98 70.5) (width 0.5) (layer "B.Cu") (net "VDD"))
 (segment (start 103.775 69) (end 104.275 68.5) (width 0.5) (layer "B.Cu") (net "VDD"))
 (segment (start 99.38 64.5) (end 97.405 66.475) (width 0.5) (layer "B.Cu") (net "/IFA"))
 (segment (start 99.914214 64.5) (end 99.38 64.5) (width 0.5) (layer "B.Cu") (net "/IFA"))
 (segment (start 104.55 64.5) (end 99.914214 64.5) (width 0.5) (layer "B.Cu") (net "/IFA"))
 (segment (start 94.050184 60.3) (end 93.595 60.755184) (width 0.5) (layer "B.Cu") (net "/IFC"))
 (segment (start 104.35 60.3) (end 104.55 60.5) (width 0.5) (layer "B.Cu") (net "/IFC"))
 (segment (start 93.595 60.755184) (end 93.595 61.525) (width 0.5) (layer "B.Cu") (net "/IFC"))
 (segment (start 94.050184 60.3) (end 104.35 60.3) (width 0.5) (layer "B.Cu") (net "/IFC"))
 (segment (start 97.215786 65.25) (end 99.965786 62.5) (width 0.5) (layer "B.Cu") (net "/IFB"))
 (segment (start 94.050184 65.25) (end 97.215786 65.25) (width 0.5) (layer "B.Cu") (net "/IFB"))
 (segment (start 93.595 66.475) (end 93.595 65.705184) (width 0.5) (layer "B.Cu") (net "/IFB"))
 (segment (start 93.595 65.705184) (end 94.050184 65.25) (width 0.5) (layer "B.Cu") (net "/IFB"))
 (segment (start 99.965786 62.5) (end 104.55 62.5) (width 0.5) (layer "B.Cu") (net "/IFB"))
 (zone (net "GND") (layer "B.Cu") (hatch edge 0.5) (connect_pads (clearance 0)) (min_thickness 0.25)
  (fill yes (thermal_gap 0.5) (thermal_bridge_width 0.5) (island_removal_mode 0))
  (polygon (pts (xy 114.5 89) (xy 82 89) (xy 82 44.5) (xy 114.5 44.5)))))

